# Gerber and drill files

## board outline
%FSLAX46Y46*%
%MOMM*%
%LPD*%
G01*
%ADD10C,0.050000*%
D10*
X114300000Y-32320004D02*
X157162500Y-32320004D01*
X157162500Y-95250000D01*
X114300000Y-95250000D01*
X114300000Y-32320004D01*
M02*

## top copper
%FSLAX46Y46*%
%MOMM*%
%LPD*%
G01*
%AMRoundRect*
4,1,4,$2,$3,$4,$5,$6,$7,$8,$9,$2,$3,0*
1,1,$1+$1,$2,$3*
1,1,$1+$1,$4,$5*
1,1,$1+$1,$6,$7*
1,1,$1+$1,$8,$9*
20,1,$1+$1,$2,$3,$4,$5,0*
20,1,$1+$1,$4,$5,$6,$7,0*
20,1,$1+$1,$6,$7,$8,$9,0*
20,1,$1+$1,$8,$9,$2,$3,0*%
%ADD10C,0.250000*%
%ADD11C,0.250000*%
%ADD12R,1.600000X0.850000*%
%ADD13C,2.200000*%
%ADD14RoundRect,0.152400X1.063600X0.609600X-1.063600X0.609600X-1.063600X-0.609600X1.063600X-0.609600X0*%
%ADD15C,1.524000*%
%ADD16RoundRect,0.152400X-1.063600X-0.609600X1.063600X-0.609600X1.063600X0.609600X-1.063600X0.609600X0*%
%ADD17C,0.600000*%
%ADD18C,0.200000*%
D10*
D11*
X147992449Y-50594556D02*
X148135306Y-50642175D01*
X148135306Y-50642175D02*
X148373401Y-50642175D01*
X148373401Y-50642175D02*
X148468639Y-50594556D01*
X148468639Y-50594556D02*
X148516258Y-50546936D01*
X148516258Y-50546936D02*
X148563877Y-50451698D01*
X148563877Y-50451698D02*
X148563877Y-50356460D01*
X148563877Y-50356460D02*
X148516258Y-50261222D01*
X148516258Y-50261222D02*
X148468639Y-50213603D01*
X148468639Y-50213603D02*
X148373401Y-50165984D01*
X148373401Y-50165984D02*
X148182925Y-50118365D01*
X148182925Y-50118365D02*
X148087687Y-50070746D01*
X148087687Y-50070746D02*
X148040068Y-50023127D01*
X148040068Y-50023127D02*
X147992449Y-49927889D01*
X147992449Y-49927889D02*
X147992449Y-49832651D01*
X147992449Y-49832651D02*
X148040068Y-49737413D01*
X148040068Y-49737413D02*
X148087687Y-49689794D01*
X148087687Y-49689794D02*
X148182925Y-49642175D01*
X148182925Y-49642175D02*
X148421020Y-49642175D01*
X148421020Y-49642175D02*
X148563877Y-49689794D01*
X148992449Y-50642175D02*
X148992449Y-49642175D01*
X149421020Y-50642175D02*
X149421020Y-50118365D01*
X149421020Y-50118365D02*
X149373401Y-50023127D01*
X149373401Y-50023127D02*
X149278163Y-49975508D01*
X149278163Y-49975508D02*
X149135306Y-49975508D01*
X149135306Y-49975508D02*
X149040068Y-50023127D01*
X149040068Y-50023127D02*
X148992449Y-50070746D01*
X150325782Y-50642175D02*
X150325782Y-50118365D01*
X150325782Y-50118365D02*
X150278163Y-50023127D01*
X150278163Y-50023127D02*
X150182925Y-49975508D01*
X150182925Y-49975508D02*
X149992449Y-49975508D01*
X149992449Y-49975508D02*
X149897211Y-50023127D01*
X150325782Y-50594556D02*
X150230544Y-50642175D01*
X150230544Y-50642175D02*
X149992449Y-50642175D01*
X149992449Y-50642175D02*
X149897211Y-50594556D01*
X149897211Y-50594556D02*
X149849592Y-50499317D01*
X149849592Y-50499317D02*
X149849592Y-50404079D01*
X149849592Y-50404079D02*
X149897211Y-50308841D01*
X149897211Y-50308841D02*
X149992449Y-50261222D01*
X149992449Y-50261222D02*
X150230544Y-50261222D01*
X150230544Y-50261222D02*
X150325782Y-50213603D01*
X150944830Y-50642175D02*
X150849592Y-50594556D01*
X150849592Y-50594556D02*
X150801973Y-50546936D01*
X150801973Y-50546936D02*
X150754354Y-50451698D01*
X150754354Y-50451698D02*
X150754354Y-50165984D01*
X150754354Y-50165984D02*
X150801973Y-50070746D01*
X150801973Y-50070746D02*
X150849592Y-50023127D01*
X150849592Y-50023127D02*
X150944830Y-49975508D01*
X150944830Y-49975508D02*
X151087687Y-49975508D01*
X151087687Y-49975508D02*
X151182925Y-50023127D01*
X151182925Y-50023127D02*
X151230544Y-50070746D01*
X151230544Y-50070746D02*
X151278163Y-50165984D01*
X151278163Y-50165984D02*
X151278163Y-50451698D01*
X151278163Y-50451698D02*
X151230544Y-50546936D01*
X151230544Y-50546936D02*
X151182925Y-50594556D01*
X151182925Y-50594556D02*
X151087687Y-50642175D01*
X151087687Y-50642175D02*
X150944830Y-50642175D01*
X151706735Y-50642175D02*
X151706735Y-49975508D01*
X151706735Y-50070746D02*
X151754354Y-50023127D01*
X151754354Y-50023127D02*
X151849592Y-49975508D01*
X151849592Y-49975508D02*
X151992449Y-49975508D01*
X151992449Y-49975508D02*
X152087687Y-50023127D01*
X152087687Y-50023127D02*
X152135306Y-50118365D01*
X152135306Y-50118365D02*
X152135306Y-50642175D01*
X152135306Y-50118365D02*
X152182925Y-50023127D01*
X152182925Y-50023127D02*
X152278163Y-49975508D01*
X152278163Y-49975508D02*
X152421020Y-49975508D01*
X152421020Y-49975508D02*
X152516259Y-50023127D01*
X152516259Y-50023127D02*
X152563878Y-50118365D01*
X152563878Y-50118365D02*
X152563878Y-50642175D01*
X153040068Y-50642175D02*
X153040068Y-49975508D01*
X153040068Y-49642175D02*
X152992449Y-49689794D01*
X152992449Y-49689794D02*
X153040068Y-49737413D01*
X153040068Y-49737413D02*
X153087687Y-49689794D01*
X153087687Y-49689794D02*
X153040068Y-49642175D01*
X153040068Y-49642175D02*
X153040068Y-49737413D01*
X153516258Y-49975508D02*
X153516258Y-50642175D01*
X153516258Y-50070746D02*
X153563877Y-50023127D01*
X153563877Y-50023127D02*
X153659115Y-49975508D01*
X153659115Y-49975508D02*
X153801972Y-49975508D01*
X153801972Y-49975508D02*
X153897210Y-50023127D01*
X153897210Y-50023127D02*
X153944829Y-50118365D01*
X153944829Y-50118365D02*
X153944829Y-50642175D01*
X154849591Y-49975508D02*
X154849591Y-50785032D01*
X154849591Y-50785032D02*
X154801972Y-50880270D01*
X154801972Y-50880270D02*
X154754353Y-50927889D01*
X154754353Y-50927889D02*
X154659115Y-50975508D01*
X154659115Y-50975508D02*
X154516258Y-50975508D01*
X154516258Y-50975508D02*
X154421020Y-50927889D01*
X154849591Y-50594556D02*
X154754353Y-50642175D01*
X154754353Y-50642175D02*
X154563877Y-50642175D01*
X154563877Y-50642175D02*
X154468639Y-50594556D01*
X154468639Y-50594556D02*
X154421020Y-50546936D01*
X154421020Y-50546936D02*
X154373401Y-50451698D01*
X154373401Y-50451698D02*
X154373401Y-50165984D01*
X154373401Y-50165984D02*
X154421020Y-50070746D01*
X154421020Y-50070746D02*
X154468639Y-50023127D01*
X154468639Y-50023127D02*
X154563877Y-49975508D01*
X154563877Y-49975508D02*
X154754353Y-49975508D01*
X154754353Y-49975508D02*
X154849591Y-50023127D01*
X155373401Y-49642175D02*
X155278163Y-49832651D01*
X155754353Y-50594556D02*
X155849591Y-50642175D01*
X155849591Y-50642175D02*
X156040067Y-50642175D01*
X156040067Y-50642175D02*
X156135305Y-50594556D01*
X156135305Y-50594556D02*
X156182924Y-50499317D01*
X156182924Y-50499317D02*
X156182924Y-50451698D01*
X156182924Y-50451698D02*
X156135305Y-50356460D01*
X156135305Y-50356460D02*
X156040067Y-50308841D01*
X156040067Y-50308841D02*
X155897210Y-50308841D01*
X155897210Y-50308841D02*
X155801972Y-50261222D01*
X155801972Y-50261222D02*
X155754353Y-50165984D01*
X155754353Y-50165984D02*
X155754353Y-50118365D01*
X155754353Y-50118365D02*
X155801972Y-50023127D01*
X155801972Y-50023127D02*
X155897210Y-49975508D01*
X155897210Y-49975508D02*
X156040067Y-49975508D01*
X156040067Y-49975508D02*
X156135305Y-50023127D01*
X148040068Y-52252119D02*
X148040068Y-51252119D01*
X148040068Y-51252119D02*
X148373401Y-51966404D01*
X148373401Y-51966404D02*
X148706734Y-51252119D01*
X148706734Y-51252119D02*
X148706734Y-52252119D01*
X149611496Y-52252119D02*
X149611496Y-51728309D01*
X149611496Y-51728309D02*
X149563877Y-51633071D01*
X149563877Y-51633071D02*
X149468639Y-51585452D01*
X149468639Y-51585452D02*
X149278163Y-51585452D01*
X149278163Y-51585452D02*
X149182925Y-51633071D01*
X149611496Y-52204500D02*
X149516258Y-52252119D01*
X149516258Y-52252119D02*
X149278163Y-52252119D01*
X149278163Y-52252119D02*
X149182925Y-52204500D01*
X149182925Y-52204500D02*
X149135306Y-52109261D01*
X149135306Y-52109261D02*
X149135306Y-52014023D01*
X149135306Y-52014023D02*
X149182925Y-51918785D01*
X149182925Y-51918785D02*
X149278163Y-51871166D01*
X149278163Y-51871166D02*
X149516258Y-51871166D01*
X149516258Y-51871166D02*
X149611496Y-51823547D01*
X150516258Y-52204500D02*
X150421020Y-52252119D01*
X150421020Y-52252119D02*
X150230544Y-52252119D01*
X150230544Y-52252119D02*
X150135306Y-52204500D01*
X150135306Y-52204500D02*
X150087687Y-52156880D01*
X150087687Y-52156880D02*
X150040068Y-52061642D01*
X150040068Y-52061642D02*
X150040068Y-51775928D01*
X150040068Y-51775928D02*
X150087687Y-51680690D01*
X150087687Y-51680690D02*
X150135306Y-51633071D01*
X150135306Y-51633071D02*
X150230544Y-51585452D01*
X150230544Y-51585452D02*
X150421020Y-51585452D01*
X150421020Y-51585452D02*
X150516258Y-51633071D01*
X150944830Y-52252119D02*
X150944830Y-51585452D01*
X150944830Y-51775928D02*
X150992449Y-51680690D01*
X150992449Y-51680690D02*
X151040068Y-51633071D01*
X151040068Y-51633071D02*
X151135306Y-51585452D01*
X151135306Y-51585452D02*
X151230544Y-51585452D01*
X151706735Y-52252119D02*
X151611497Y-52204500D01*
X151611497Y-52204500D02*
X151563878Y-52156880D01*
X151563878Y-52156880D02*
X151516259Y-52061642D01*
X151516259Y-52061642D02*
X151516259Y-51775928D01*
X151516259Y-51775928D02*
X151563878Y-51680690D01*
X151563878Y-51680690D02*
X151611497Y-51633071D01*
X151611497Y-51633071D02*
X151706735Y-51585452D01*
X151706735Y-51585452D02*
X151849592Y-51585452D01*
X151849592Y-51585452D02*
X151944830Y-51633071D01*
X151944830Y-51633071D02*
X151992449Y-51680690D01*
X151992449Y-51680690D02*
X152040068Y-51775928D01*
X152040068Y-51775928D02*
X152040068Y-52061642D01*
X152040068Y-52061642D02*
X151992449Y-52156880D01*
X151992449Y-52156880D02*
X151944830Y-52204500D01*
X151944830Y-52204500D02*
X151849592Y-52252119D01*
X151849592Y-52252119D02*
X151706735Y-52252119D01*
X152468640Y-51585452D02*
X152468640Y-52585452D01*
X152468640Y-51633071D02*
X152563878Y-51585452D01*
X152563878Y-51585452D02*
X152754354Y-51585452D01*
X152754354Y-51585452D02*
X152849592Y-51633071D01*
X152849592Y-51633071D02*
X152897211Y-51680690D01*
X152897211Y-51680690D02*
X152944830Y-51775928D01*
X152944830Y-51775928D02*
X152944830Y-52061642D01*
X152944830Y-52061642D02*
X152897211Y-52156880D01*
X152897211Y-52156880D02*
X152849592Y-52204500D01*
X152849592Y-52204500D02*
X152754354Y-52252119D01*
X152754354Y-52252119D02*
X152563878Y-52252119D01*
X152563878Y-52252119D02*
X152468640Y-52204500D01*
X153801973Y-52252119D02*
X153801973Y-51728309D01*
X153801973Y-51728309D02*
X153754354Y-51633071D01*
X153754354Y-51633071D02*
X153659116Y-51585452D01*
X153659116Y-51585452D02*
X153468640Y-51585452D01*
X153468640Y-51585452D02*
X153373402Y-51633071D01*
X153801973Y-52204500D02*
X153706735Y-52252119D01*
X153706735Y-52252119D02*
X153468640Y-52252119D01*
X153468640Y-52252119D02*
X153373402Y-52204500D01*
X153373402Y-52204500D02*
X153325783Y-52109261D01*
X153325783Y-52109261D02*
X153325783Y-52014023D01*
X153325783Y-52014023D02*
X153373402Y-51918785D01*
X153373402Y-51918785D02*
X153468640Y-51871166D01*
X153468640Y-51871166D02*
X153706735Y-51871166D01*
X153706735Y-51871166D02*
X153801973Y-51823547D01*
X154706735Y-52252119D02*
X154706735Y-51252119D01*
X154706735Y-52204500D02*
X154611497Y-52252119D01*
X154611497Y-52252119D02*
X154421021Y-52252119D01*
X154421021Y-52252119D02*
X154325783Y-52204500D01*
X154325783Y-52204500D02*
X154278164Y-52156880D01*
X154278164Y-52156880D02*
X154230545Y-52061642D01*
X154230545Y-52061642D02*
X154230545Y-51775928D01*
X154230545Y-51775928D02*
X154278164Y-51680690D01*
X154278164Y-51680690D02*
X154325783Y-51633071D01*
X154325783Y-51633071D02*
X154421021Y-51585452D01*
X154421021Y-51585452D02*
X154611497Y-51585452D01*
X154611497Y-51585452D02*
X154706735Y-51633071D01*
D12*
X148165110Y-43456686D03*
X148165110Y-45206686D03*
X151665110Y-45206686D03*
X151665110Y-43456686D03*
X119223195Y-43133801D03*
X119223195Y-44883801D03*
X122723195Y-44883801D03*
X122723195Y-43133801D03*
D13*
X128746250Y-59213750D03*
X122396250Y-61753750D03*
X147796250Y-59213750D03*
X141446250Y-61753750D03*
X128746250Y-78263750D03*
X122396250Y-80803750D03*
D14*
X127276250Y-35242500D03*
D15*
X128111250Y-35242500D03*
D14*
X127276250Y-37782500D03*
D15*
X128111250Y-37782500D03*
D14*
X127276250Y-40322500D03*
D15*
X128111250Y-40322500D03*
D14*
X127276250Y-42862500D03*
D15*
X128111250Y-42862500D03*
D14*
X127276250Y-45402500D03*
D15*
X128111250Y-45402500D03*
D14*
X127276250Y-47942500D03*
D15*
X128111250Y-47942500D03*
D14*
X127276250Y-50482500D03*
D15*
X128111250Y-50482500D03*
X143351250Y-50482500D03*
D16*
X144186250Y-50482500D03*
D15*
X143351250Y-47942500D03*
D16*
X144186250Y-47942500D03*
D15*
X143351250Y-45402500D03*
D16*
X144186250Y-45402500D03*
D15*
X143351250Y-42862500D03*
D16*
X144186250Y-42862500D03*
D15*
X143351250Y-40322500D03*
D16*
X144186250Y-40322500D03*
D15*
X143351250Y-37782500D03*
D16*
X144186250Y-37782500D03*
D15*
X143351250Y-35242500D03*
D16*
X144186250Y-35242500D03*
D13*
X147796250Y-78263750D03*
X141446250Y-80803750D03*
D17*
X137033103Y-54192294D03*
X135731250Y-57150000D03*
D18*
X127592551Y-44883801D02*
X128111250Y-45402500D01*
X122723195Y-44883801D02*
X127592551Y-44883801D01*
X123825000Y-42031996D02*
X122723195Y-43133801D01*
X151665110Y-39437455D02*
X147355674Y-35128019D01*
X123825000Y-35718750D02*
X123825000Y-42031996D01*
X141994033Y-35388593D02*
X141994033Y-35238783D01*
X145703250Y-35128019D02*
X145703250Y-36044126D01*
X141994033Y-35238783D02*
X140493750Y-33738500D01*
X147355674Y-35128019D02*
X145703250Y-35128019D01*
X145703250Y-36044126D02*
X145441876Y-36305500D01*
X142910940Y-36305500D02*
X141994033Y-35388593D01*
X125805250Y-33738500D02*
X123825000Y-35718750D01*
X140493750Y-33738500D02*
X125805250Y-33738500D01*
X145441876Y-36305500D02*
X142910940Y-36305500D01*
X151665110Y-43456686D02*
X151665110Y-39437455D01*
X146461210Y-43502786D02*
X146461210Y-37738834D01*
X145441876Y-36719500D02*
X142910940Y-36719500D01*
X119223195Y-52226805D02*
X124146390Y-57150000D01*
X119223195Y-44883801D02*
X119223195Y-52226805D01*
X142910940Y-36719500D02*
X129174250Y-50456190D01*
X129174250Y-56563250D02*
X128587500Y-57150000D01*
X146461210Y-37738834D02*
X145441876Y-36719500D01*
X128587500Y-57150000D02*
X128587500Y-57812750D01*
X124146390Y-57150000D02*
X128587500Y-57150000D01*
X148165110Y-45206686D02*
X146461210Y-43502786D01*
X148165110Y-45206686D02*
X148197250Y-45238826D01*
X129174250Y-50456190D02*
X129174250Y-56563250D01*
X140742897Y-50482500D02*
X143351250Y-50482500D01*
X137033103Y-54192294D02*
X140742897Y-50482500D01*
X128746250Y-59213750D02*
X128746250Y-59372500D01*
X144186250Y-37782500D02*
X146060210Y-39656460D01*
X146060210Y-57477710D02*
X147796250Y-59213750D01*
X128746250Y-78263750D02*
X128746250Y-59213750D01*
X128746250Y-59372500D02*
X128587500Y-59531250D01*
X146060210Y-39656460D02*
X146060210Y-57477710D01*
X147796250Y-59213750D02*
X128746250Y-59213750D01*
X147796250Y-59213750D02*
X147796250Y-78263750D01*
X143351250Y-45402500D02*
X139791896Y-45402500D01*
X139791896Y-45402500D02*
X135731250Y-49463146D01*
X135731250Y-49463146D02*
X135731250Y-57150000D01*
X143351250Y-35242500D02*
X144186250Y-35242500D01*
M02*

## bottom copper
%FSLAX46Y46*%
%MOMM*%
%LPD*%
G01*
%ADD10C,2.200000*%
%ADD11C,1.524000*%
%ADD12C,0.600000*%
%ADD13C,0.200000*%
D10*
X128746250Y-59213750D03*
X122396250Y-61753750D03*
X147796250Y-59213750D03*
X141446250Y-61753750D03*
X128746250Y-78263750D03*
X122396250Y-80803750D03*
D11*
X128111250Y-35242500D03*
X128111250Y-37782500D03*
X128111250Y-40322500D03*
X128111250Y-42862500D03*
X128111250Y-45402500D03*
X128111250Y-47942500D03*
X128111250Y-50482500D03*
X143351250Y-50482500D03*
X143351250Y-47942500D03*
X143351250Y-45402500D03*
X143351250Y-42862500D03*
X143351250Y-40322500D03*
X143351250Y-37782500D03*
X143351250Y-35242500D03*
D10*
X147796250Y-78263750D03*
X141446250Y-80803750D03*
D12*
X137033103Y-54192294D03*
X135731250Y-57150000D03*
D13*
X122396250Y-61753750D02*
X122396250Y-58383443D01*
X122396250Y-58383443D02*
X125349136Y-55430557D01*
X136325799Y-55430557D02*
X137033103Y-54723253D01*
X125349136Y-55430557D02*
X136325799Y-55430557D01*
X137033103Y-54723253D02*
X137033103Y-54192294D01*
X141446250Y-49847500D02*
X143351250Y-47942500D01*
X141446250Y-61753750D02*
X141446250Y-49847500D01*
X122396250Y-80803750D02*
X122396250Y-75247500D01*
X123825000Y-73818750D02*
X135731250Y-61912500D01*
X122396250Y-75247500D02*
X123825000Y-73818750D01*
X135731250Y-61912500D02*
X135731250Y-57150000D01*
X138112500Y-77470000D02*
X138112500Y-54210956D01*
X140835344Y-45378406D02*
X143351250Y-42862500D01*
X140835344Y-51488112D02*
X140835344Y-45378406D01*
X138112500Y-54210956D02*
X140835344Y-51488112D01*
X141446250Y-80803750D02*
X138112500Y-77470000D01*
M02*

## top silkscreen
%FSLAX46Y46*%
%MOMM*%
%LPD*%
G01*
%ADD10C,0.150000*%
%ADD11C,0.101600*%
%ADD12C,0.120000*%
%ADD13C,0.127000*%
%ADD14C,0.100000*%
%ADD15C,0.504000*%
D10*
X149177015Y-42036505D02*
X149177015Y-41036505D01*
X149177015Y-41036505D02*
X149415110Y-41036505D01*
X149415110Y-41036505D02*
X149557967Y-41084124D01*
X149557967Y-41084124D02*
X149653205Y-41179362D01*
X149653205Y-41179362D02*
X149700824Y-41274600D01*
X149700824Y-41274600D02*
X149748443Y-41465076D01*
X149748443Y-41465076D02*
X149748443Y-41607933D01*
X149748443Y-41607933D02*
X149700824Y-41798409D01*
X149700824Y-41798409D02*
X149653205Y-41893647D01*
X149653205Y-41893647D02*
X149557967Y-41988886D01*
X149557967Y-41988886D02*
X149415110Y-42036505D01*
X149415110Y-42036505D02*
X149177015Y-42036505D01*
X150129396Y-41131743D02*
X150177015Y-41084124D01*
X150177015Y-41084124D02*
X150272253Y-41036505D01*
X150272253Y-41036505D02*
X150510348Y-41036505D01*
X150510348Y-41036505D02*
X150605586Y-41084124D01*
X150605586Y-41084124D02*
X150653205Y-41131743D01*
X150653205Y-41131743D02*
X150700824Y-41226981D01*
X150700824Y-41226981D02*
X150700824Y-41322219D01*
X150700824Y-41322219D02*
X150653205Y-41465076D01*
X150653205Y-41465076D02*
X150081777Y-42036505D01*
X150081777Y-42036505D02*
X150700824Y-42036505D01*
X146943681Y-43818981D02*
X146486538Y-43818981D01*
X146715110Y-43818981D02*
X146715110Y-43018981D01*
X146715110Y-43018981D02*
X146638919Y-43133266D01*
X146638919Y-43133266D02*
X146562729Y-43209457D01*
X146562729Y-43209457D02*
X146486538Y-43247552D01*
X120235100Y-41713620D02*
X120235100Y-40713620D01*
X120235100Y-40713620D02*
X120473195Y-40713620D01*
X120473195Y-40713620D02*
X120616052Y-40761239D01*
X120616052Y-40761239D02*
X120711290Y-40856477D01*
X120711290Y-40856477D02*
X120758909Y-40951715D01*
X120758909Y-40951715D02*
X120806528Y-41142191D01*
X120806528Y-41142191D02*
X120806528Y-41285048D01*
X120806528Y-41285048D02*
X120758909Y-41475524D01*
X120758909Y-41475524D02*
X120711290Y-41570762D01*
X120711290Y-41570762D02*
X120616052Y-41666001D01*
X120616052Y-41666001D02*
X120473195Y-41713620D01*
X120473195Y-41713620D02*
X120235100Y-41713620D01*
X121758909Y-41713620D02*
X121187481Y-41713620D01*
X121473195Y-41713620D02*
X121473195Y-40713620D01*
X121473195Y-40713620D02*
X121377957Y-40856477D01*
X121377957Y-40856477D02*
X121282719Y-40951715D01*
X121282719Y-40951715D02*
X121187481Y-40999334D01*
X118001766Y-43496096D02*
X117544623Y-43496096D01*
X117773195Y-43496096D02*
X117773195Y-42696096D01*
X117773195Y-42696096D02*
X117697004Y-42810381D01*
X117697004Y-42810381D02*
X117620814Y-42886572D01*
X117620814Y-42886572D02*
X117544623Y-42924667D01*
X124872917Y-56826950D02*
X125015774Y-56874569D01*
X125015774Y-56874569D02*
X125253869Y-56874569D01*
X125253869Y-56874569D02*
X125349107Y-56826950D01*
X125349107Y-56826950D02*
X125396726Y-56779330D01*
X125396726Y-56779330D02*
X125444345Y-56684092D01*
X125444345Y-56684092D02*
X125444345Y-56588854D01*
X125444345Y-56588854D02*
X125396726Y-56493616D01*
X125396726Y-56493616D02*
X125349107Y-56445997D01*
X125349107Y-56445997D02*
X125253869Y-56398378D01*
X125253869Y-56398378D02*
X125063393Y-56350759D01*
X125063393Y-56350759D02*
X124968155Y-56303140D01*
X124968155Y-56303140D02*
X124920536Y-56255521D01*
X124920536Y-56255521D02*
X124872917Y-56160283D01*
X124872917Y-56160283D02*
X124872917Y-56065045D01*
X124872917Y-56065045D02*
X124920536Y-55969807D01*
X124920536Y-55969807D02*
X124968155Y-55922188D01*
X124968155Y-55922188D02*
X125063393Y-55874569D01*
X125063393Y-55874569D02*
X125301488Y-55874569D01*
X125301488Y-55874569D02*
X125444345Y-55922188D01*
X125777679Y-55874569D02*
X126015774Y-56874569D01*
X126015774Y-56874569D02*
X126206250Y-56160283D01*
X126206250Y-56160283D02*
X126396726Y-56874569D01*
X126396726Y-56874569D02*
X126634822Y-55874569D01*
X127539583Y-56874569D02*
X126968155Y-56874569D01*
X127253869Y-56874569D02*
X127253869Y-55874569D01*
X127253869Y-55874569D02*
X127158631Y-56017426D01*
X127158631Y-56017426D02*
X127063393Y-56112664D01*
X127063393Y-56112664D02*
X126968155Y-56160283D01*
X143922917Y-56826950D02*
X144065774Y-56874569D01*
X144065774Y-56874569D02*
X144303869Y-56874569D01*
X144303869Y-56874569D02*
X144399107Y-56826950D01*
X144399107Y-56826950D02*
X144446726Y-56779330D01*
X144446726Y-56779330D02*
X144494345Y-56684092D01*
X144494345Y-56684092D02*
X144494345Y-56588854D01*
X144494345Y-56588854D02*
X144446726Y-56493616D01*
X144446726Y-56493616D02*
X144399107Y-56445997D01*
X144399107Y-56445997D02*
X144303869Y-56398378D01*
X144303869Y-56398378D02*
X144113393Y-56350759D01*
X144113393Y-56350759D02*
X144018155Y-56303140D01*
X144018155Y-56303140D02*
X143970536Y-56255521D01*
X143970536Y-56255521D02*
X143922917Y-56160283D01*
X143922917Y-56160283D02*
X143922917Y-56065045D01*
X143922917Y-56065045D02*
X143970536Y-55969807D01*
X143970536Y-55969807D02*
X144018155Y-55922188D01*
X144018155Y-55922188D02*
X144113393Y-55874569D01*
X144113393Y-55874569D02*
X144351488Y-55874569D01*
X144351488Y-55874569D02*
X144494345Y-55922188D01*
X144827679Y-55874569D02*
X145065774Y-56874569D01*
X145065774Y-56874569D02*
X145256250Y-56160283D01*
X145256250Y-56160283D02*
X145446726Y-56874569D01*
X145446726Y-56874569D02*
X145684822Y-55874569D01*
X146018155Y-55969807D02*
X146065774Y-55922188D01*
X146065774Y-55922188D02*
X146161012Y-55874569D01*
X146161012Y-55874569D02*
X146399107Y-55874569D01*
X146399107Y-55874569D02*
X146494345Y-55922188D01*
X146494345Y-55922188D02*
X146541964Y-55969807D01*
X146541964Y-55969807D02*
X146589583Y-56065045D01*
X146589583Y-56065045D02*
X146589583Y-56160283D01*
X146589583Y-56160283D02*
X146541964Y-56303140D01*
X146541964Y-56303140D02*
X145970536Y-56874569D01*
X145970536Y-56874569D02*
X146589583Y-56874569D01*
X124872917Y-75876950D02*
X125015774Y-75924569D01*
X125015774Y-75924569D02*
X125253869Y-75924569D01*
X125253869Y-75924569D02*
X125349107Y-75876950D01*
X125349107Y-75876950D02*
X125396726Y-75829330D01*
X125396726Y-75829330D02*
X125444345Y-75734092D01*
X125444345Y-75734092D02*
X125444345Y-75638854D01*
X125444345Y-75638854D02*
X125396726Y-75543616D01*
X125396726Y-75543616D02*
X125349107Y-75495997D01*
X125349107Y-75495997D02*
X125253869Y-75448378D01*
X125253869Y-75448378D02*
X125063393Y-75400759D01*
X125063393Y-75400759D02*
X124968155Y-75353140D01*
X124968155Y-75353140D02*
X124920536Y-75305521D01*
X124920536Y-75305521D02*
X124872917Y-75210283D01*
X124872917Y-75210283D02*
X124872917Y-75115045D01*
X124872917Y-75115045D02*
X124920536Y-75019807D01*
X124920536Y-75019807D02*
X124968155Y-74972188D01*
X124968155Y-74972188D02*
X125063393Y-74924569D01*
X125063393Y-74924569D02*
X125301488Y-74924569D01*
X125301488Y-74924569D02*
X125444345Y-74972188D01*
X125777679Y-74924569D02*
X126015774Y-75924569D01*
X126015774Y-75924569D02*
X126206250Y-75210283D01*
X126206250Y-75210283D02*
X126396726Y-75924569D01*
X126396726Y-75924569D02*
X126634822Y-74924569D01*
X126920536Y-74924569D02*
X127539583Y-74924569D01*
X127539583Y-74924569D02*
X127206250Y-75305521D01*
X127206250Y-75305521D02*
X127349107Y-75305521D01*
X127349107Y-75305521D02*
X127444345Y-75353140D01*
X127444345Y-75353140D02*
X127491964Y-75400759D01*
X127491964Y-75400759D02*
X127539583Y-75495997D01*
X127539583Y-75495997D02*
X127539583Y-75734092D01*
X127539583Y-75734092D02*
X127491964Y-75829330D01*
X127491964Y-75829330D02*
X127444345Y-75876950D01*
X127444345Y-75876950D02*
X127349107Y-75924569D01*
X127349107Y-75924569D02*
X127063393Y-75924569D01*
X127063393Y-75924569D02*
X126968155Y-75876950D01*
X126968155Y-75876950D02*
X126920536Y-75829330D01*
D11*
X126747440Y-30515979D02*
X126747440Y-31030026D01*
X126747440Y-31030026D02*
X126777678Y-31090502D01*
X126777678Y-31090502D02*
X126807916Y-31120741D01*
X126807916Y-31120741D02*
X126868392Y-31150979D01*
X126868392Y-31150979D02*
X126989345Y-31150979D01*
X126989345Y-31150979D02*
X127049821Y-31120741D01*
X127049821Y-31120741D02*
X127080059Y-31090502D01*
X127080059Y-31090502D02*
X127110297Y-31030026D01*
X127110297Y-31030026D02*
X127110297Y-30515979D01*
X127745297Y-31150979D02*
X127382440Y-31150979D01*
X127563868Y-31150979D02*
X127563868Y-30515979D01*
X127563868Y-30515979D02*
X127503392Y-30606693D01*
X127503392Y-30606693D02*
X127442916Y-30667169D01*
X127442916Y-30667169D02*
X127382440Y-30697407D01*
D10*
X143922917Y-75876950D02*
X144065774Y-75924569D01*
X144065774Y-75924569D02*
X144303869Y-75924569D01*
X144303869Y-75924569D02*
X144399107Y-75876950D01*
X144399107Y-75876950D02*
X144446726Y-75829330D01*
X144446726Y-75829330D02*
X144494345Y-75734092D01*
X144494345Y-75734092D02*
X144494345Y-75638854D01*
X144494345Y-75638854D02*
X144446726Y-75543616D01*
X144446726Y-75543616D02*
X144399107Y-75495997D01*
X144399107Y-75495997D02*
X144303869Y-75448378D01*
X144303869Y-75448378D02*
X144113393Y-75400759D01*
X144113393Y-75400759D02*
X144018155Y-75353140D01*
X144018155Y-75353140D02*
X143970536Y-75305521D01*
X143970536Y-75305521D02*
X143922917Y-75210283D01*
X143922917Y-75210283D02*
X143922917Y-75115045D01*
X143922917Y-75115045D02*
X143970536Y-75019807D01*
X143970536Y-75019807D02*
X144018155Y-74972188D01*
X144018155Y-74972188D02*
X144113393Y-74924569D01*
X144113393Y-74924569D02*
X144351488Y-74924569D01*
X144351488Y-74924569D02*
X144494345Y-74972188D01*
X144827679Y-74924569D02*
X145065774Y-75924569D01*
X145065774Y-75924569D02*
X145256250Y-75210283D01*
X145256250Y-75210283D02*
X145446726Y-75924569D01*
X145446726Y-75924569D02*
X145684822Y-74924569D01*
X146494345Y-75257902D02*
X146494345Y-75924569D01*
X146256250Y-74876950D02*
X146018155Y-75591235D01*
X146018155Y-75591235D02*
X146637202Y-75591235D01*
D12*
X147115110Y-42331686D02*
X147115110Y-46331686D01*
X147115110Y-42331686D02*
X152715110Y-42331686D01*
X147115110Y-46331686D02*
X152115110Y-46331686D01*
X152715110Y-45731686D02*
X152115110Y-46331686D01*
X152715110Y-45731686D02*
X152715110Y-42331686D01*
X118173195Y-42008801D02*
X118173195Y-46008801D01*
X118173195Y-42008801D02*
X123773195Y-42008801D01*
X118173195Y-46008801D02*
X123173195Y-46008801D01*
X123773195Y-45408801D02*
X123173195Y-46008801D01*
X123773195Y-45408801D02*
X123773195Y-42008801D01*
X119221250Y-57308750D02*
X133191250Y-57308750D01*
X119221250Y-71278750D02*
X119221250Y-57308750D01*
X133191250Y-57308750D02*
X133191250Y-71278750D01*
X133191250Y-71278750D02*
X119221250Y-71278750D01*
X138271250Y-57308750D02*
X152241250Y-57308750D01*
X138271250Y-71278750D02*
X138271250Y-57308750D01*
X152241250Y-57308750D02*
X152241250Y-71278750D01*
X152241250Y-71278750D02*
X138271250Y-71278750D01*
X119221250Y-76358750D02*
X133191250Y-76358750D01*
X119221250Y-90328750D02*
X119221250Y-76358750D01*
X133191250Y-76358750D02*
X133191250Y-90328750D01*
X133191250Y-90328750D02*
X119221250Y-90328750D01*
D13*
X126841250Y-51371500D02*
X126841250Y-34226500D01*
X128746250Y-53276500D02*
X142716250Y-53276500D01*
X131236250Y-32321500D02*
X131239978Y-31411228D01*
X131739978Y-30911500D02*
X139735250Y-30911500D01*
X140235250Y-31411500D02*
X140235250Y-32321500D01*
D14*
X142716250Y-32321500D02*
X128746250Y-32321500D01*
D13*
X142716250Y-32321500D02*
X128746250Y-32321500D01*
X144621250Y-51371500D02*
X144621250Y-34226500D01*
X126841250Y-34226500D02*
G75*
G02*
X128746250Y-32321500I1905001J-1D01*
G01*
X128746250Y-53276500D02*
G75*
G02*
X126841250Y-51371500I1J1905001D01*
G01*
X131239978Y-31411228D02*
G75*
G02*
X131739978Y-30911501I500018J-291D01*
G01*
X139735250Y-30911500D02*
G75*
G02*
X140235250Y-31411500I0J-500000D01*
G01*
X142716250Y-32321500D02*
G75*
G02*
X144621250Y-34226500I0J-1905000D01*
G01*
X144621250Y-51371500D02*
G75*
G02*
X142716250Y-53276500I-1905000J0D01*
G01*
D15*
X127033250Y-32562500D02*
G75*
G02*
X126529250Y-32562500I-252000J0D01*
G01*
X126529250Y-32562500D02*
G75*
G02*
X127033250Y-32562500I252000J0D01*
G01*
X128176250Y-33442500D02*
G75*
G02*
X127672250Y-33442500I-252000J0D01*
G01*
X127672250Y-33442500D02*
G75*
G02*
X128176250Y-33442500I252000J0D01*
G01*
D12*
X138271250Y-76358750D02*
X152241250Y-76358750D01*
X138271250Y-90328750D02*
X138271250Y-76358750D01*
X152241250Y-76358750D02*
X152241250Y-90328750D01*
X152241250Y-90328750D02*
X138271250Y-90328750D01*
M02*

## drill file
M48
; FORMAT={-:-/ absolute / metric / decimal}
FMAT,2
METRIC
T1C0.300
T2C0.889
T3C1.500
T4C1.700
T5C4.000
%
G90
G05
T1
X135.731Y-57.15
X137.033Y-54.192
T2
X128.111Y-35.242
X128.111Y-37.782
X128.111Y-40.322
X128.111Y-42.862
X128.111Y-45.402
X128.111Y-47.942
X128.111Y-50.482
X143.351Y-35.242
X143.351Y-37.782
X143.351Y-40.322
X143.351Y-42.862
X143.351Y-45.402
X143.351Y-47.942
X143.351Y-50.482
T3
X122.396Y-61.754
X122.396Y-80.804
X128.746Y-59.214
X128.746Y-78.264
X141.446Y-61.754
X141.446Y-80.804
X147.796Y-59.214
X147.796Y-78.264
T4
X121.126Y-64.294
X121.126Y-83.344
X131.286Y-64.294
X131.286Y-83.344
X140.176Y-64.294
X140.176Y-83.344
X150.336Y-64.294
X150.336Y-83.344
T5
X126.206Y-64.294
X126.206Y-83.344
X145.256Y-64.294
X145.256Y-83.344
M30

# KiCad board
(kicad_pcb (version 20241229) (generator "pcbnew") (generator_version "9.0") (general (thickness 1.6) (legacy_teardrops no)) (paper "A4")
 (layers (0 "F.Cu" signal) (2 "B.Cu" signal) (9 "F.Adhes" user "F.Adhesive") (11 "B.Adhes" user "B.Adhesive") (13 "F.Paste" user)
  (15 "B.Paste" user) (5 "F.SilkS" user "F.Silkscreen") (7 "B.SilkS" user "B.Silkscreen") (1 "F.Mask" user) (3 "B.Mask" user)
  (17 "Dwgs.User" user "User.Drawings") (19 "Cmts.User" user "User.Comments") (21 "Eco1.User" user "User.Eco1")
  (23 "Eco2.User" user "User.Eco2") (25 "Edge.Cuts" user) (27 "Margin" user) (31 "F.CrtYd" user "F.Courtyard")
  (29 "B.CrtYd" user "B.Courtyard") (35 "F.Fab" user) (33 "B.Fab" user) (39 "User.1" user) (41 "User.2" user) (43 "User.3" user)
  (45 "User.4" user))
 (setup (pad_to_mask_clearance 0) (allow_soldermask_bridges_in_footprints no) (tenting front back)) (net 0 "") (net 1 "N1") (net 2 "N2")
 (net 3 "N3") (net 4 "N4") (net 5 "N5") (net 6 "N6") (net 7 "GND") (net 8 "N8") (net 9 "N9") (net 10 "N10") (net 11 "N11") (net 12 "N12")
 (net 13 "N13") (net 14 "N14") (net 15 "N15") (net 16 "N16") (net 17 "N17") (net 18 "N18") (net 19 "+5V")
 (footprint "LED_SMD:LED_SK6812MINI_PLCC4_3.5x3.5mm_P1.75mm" (layer "F.Cu") (at 149.91511 44.331686)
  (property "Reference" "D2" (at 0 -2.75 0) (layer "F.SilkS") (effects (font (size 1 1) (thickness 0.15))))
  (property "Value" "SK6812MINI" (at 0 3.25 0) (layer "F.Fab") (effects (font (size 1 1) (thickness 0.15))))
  (fp_line (start -2.8 -2) (end -2.8 2) (stroke (width 0.12) (type default)) (layer "F.SilkS"))
  (fp_line (start -2.8 -2) (end 2.8 -2) (stroke (width 0.12) (type solid)) (layer "F.SilkS"))
  (fp_line (start -2.8 2) (end 2.2 2) (stroke (width 0.12) (type solid)) (layer "F.SilkS"))
  (fp_line (start 2.8 1.4) (end 2.2 2) (stroke (width 0.12) (type default)) (layer "F.SilkS"))
  (fp_line (start 2.8 1.4) (end 2.8 -2) (stroke (width 0.12) (type solid)) (layer "F.SilkS"))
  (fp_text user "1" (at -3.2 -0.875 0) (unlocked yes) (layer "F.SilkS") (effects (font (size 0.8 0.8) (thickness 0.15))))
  (pad "1" smd rect (at -1.75 -0.875) (size 1.6 0.85) (layers "F.Cu" "F.Mask" "F.Paste") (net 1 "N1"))
  (pad "2" smd rect (at -1.75 0.875) (size 1.6 0.85) (layers "F.Cu" "F.Mask" "F.Paste") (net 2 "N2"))
  (pad "3" smd rect (at 1.75 0.875) (size 1.6 0.85) (layers "F.Cu" "F.Mask" "F.Paste") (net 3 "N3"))
  (pad "4" smd rect (at 1.75 -0.875) (size 1.6 0.85) (layers "F.Cu" "F.Mask" "F.Paste") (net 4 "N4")))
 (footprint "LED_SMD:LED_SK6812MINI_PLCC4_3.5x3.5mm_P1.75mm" (layer "F.Cu") (at 120.973195 44.008801)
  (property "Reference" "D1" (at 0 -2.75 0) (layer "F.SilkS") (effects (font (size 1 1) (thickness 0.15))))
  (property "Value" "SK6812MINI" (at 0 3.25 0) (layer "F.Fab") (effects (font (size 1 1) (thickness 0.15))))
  (fp_line (start -2.8 -2) (end -2.8 2) (stroke (width 0.12) (type default)) (layer "F.SilkS"))
  (fp_line (start -2.8 -2) (end 2.8 -2) (stroke (width 0.12) (type solid)) (layer "F.SilkS"))
  (fp_line (start -2.8 2) (end 2.2 2) (stroke (width 0.12) (type solid)) (layer "F.SilkS"))
  (fp_line (start 2.8 1.4) (end 2.2 2) (stroke (width 0.12) (type default)) (layer "F.SilkS"))
  (fp_line (start 2.8 1.4) (end 2.8 -2) (stroke (width 0.12) (type solid)) (layer "F.SilkS"))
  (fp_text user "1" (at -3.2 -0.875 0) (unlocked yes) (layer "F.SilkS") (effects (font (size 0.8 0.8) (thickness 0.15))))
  (pad "1" smd rect (at -1.75 -0.875) (size 1.6 0.85) (layers "F.Cu" "F.Mask" "F.Paste") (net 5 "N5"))
  (pad "2" smd rect (at -1.75 0.875) (size 1.6 0.85) (layers "F.Cu" "F.Mask" "F.Paste") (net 2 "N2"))
  (pad "3" smd rect (at 1.75 0.875) (size 1.6 0.85) (layers "F.Cu" "F.Mask" "F.Paste") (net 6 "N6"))
  (pad "4" smd rect (at 1.75 -0.875) (size 1.6 0.85) (layers "F.Cu" "F.Mask" "F.Paste") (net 4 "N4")))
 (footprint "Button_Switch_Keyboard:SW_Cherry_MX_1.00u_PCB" (layer "F.Cu") (at 128.74625 59.21375)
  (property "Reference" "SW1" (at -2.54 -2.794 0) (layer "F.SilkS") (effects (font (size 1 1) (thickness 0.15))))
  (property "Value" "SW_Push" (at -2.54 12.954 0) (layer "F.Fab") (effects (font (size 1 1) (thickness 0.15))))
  (fp_line (start -9.525 -1.905) (end 4.445 -1.905) (stroke (width 0.12) (type solid)) (layer "F.SilkS"))
  (fp_line (start -9.525 12.065) (end -9.525 -1.905) (stroke (width 0.12) (type solid)) (layer "F.SilkS"))
  (fp_line (start 4.445 -1.905) (end 4.445 12.065) (stroke (width 0.12) (type solid)) (layer "F.SilkS"))
  (fp_line (start 4.445 12.065) (end -9.525 12.065) (stroke (width 0.12) (type solid)) (layer "F.SilkS"))
  (pad "" np_thru_hole circle (at -7.62 5.08) (size 1.7 1.7) (drill 1.7) (layers "*.Cu" "*.Mask"))
  (pad "" np_thru_hole circle (at -2.54 5.08) (size 4 4) (drill 4) (layers "*.Cu" "*.Mask"))
  (pad "" np_thru_hole circle (at 2.54 5.08) (size 1.7 1.7) (drill 1.7) (layers "*.Cu" "*.Mask"))
  (pad "1" thru_hole circle (at 0 0) (size 2.2 2.2) (drill 1.5) (layers "*.Cu" "*.Mask") (remove_unused_layers no) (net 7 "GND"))
  (pad "2" thru_hole circle (at -6.35 2.54) (size 2.2 2.2) (drill 1.5) (layers "*.Cu" "*.Mask") (remove_unused_layers no) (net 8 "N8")))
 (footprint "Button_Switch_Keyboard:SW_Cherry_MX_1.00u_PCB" (layer "F.Cu") (at 147.79625 59.21375)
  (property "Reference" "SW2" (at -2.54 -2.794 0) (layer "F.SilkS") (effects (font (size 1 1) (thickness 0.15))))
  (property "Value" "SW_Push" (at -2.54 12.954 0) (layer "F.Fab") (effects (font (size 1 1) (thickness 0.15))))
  (fp_line (start -9.525 -1.905) (end 4.445 -1.905) (stroke (width 0.12) (type solid)) (layer "F.SilkS"))
  (fp_line (start -9.525 12.065) (end -9.525 -1.905) (stroke (width 0.12) (type solid)) (layer "F.SilkS"))
  (fp_line (start 4.445 -1.905) (end 4.445 12.065) (stroke (width 0.12) (type solid)) (layer "F.SilkS"))
  (fp_line (start 4.445 12.065) (end -9.525 12.065) (stroke (width 0.12) (type solid)) (layer "F.SilkS"))
  (pad "" np_thru_hole circle (at -7.62 5.08) (size 1.7 1.7) (drill 1.7) (layers "*.Cu" "*.Mask"))
  (pad "" np_thru_hole circle (at -2.54 5.08) (size 4 4) (drill 4) (layers "*.Cu" "*.Mask"))
  (pad "" np_thru_hole circle (at 2.54 5.08) (size 1.7 1.7) (drill 1.7) (layers "*.Cu" "*.Mask"))
  (pad "1" thru_hole circle (at 0 0) (size 2.2 2.2) (drill 1.5) (layers "*.Cu" "*.Mask") (remove_unused_layers no) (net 7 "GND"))
  (pad "2" thru_hole circle (at -6.35 2.54) (size 2.2 2.2) (drill 1.5) (layers "*.Cu" "*.Mask") (remove_unused_layers no) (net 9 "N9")))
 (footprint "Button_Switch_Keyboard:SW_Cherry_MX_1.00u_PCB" (layer "F.Cu") (at 128.74625 78.26375)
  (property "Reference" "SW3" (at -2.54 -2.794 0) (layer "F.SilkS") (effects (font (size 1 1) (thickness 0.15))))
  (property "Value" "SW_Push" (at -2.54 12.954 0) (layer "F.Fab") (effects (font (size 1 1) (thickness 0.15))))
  (fp_line (start -9.525 -1.905) (end 4.445 -1.905) (stroke (width 0.12) (type solid)) (layer "F.SilkS"))
  (fp_line (start -9.525 12.065) (end -9.525 -1.905) (stroke (width 0.12) (type solid)) (layer "F.SilkS"))
  (fp_line (start 4.445 -1.905) (end 4.445 12.065) (stroke (width 0.12) (type solid)) (layer "F.SilkS"))
  (fp_line (start 4.445 12.065) (end -9.525 12.065) (stroke (width 0.12) (type solid)) (layer "F.SilkS"))
  (pad "" np_thru_hole circle (at -7.62 5.08) (size 1.7 1.7) (drill 1.7) (layers "*.Cu" "*.Mask"))
  (pad "" np_thru_hole circle (at -2.54 5.08) (size 4 4) (drill 4) (layers "*.Cu" "*.Mask"))
  (pad "" np_thru_hole circle (at 2.54 5.08) (size 1.7 1.7) (drill 1.7) (layers "*.Cu" "*.Mask"))
  (pad "1" thru_hole circle (at 0 0) (size 2.2 2.2) (drill 1.5) (layers "*.Cu" "*.Mask") (remove_unused_layers no) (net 7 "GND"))
  (pad "2" thru_hole circle (at -6.35 2.54) (size 2.2 2.2) (drill 1.5) (layers "*.Cu" "*.Mask") (remove_unused_layers no) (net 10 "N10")))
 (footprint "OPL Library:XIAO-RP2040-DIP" (layer "F.Cu") (at 135.73125 42.8625)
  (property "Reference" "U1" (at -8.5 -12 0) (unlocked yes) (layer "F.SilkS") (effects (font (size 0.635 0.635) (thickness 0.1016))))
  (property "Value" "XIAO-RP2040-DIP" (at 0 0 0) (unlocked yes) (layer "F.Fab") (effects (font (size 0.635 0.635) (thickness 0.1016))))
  (fp_line (start -8.89 8.509) (end -8.89 -8.636) (stroke (width 0.127) (type solid)) (layer "F.SilkS"))
  (fp_line (start -6.985 10.414) (end 6.985 10.414) (stroke (width 0.127) (type solid)) (layer "F.SilkS"))
  (fp_line (start -4.495 -10.541) (end -4.491272 -11.451272) (stroke (width 0.127) (type solid)) (layer "F.SilkS"))
  (fp_line (start -3.991272 -11.951) (end 4.004 -11.951) (stroke (width 0.127) (type solid)) (layer "F.SilkS"))
  (fp_line (start 4.504 -11.451) (end 4.504 -10.541) (stroke (width 0.127) (type solid)) (layer "F.SilkS"))
  (fp_line (start 6.985 -10.541) (end -6.985 -10.541) (stroke (width 0.1) (type solid)) (layer "F.SilkS"))
  (fp_line (start 6.985 -10.541) (end -6.985 -10.541) (stroke (width 0.127) (type solid)) (layer "F.SilkS"))
  (fp_line (start 8.89 8.509) (end 8.89 -8.636) (stroke (width 0.127) (type solid)) (layer "F.SilkS"))
  (fp_arc (start -8.89 -8.636) (mid -8.332038 -9.983038) (end -6.985 -10.541) (stroke (width 0.127) (type solid)) (layer "F.SilkS"))
  (fp_arc (start -6.985 10.414) (mid -8.332038 9.856038) (end -8.89 8.509) (stroke (width 0.127) (type solid)) (layer "F.SilkS"))
  (fp_arc (start -4.491272 -11.451272) (mid -4.344728 -11.80464) (end -3.991272 -11.951) (stroke (width 0.127) (type default))
   (layer "F.SilkS"))
  (fp_arc (start 4.004 -11.951) (mid 4.357553 -11.804553) (end 4.504 -11.451) (stroke (width 0.127) (type default)) (layer "F.SilkS"))
  (fp_arc (start 6.985 -10.541) (mid 8.332038 -9.983038) (end 8.89 -8.636) (stroke (width 0.127) (type solid)) (layer "F.SilkS"))
  (fp_arc (start 8.89 8.509) (mid 8.332038 9.856038) (end 6.985 10.414) (stroke (width 0.127) (type solid)) (layer "F.SilkS"))
  (fp_circle (center -8.95 -10.3) (end -8.95 -10.554) (stroke (width 0.5) (type solid)) (fill yes) (layer "F.SilkS"))
  (fp_circle (center -7.807 -9.42) (end -7.807 -9.674) (stroke (width 0.5) (type solid)) (fill yes) (layer "F.SilkS"))
  (pad "1" smd roundrect (at -8.455 -7.62 180) (size 2.432 1.524) (layers "F.Cu" "F.Mask") (roundrect_rratio 0.1) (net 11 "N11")
   (thermal_bridge_angle 45))
  (pad "1" thru_hole circle (at -7.62 -7.62 180) (size 1.524 1.524) (drill 0.889) (layers "*.Cu" "*.Mask") (remove_unused_layers no)
   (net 11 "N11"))
  (pad "2" smd roundrect (at -8.455 -5.08 180) (size 2.432 1.524) (layers "F.Cu" "F.Mask") (roundrect_rratio 0.1) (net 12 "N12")
   (thermal_bridge_angle 45))
  (pad "2" thru_hole circle (at -7.62 -5.08 180) (size 1.524 1.524) (drill 0.889) (layers "*.Cu" "*.Mask") (remove_unused_layers no)
   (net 12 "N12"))
  (pad "3" smd roundrect (at -8.455 -2.54 180) (size 2.432 1.524) (layers "F.Cu" "F.Mask") (roundrect_rratio 0.1) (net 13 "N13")
   (thermal_bridge_angle 45))
  (pad "3" thru_hole circle (at -7.62 -2.54 180) (size 1.524 1.524) (drill 0.889) (layers "*.Cu" "*.Mask") (remove_unused_layers no)
   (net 13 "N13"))
  (pad "4" smd roundrect (at -8.455 0 180) (size 2.432 1.524) (layers "F.Cu" "F.Mask") (roundrect_rratio 0.1) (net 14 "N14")
   (thermal_bridge_angle 45))
  (pad "4" thru_hole circle (at -7.62 0 180) (size 1.524 1.524) (drill 0.889) (layers "*.Cu" "*.Mask") (remove_unused_layers no)
   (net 14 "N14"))
  (pad "5" smd roundrect (at -8.455 2.54 180) (size 2.432 1.524) (layers "F.Cu" "F.Mask") (roundrect_rratio 0.1) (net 6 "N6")
   (thermal_bridge_angle 45))
  (pad "5" thru_hole circle (at -7.62 2.54 180) (size 1.524 1.524) (drill 0.889) (layers "*.Cu" "*.Mask") (remove_unused_layers no)
   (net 6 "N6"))
  (pad "6" smd roundrect (at -8.455 5.08 180) (size 2.432 1.524) (layers "F.Cu" "F.Mask") (roundrect_rratio 0.1) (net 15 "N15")
   (thermal_bridge_angle 45))
  (pad "6" thru_hole circle (at -7.62 5.08 180) (size 1.524 1.524) (drill 0.889) (layers "*.Cu" "*.Mask") (remove_unused_layers no)
   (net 15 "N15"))
  (pad "7" smd roundrect (at -8.455 7.62 180) (size 2.432 1.524) (layers "F.Cu" "F.Mask") (roundrect_rratio 0.1) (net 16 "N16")
   (thermal_bridge_angle 45))
  (pad "7" thru_hole circle (at -7.62 7.62 180) (size 1.524 1.524) (drill 0.889) (layers "*.Cu" "*.Mask") (remove_unused_layers no)
   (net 16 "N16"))
  (pad "8" thru_hole circle (at 7.62 7.62) (size 1.524 1.524) (drill 0.889) (layers "*.Cu" "*.Mask") (remove_unused_layers no) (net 8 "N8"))
  (pad "8" smd roundrect (at 8.455 7.62) (size 2.432 1.524) (layers "F.Cu" "F.Mask") (roundrect_rratio 0.1) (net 8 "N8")
   (thermal_bridge_angle 45))
  (pad "9" thru_hole circle (at 7.62 5.08) (size 1.524 1.524) (drill 0.889) (layers "*.Cu" "*.Mask") (remove_unused_layers no) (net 9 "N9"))
  (pad "9" smd roundrect (at 8.455 5.08) (size 2.432 1.524) (layers "F.Cu" "F.Mask") (roundrect_rratio 0.1) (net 9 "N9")
   (thermal_bridge_angle 45))
  (pad "10" thru_hole circle (at 7.62 2.54) (size 1.524 1.524) (drill 0.889) (layers "*.Cu" "*.Mask") (remove_unused_layers no)
   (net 10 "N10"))
  (pad "10" smd roundrect (at 8.455 2.54) (size 2.432 1.524) (layers "F.Cu" "F.Mask") (roundrect_rratio 0.1) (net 10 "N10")
   (thermal_bridge_angle 45))
  (pad "11" thru_hole circle (at 7.62 0) (size 1.524 1.524) (drill 0.889) (layers "*.Cu" "*.Mask") (remove_unused_layers no) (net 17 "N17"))
  (pad "11" smd roundrect (at 8.455 0) (size 2.432 1.524) (layers "F.Cu" "F.Mask") (roundrect_rratio 0.1) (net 17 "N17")
   (thermal_bridge_angle 45))
  (pad "12" thru_hole circle (at 7.62 -2.54) (size 1.524 1.524) (drill 0.889) (layers "*.Cu" "*.Mask") (remove_unused_layers no)
   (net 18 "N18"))
  (pad "12" smd roundrect (at 8.455 -2.54) (size 2.432 1.524) (layers "F.Cu" "F.Mask") (roundrect_rratio 0.1) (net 18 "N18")
   (thermal_bridge_angle 45))
  (pad "13" thru_hole circle (at 7.62 -5.08) (size 1.524 1.524) (drill 0.889) (layers "*.Cu" "*.Mask") (remove_unused_layers no)
   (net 7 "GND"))
  (pad "13" smd roundrect (at 8.455 -5.08) (size 2.432 1.524) (layers "F.Cu" "F.Mask") (roundrect_rratio 0.1) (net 7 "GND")
   (thermal_bridge_angle 45))
  (pad "14" thru_hole circle (at 7.62 -7.62) (size 1.524 1.524) (drill 0.889) (layers "*.Cu" "*.Mask") (remove_unused_layers no)
   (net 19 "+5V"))
  (pad "14" smd roundrect (at 8.455 -7.62) (size 2.432 1.524) (layers "F.Cu" "F.Mask") (roundrect_rratio 0.1) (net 19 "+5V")
   (thermal_bridge_angle 45)))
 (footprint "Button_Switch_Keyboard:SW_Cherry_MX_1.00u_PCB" (layer "F.Cu") (at 147.79625 78.26375)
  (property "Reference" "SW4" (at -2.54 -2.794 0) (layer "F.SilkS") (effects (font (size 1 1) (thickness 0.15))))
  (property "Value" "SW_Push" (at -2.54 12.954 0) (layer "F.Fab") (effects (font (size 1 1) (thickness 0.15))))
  (fp_line (start -9.525 -1.905) (end 4.445 -1.905) (stroke (width 0.12) (type solid)) (layer "F.SilkS"))
  (fp_line (start -9.525 12.065) (end -9.525 -1.905) (stroke (width 0.12) (type solid)) (layer "F.SilkS"))
  (fp_line (start 4.445 -1.905) (end 4.445 12.065) (stroke (width 0.12) (type solid)) (layer "F.SilkS"))
  (fp_line (start 4.445 12.065) (end -9.525 12.065) (stroke (width 0.12) (type solid)) (layer "F.SilkS"))
  (pad "" np_thru_hole circle (at -7.62 5.08) (size 1.7 1.7) (drill 1.7) (layers "*.Cu" "*.Mask"))
  (pad "" np_thru_hole circle (at -2.54 5.08) (size 4 4) (drill 4) (layers "*.Cu" "*.Mask"))
  (pad "" np_thru_hole circle (at 2.54 5.08) (size 1.7 1.7) (drill 1.7) (layers "*.Cu" "*.Mask"))
  (pad "1" thru_hole circle (at 0 0) (size 2.2 2.2) (drill 1.5) (layers "*.Cu" "*.Mask") (remove_unused_layers no) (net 7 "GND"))
  (pad "2" thru_hole circle (at -6.35 2.54) (size 2.2 2.2) (drill 1.5) (layers "*.Cu" "*.Mask") (remove_unused_layers no) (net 17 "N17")))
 (gr_rect (start 114.3 32.320004) (end 157.1625 95.25) (stroke (width 0.05) (type default)) (fill no) (layer "Edge.Cuts"))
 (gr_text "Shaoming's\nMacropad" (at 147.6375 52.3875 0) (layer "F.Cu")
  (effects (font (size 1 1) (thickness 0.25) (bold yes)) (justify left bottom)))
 (segment (start 127.592551 44.883801) (end 128.11125 45.4025) (width 0.2) (layer "F.Cu") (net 6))
 (segment (start 122.723195 44.883801) (end 127.592551 44.883801) (width 0.2) (layer "F.Cu") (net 6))
 (segment (start 123.825 42.031996) (end 122.723195 43.133801) (width 0.2) (layer "F.Cu") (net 4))
 (segment (start 151.66511 39.437455) (end 147.355674 35.128019) (width 0.2) (layer "F.Cu") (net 4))
 (segment (start 123.825 35.71875) (end 123.825 42.031996) (width 0.2) (layer "F.Cu") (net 4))
 (segment (start 141.994033 35.388593) (end 141.994033 35.238783) (width 0.2) (layer "F.Cu") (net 4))
 (segment (start 145.70325 35.128019) (end 145.70325 36.044126) (width 0.2) (layer "F.Cu") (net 4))
 (segment (start 141.994033 35.238783) (end 140.49375 33.7385) (width 0.2) (layer "F.Cu") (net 4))
 (segment (start 147.355674 35.128019) (end 145.70325 35.128019) (width 0.2) (layer "F.Cu") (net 4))
 (segment (start 145.70325 36.044126) (end 145.441876 36.3055) (width 0.2) (layer "F.Cu") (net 4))
 (segment (start 142.91094 36.3055) (end 141.994033 35.388593) (width 0.2) (layer "F.Cu") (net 4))
 (segment (start 125.80525 33.7385) (end 123.825 35.71875) (width 0.2) (layer "F.Cu") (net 4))
 (segment (start 140.49375 33.7385) (end 125.80525 33.7385) (width 0.2) (layer "F.Cu") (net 4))
 (segment (start 145.441876 36.3055) (end 142.91094 36.3055) (width 0.2) (layer "F.Cu") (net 4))
 (segment (start 151.66511 43.456686) (end 151.66511 39.437455) (width 0.2) (layer "F.Cu") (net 4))
 (segment (start 146.46121 43.502786) (end 146.46121 37.738834) (width 0.2) (layer "F.Cu") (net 2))
 (segment (start 145.441876 36.7195) (end 142.91094 36.7195) (width 0.2) (layer "F.Cu") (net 2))
 (segment (start 119.223195 52.226805) (end 124.14639 57.15) (width 0.2) (layer "F.Cu") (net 2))
 (segment (start 119.223195 44.883801) (end 119.223195 52.226805) (width 0.2) (layer "F.Cu") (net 2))
 (segment (start 142.91094 36.7195) (end 129.17425 50.45619) (width 0.2) (layer "F.Cu") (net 2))
 (segment (start 129.17425 56.56325) (end 128.5875 57.15) (width 0.2) (layer "F.Cu") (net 2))
 (segment (start 146.46121 37.738834) (end 145.441876 36.7195) (width 0.2) (layer "F.Cu") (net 2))
 (segment (start 128.5875 57.15) (end 128.5875 57.81275) (width 0.2) (layer "F.Cu") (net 2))
 (segment (start 124.14639 57.15) (end 128.5875 57.15) (width 0.2) (layer "F.Cu") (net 2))
 (segment (start 148.16511 45.206686) (end 146.46121 43.502786) (width 0.2) (layer "F.Cu") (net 2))
 (segment (start 148.16511 45.206686) (end 148.19725 45.238826) (width 0.2) (layer "F.Cu") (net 2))
 (segment (start 129.17425 50.45619) (end 129.17425 56.56325) (width 0.2) (layer "F.Cu") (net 2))
 (segment (start 140.742897 50.4825) (end 143.35125 50.4825) (width 0.2) (layer "F.Cu") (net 8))
 (segment (start 137.033103 54.192294) (end 140.742897 50.4825) (width 0.2) (layer "F.Cu") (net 8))
 (via (at 137.033103 54.192294) (size 0.6) (drill 0.3) (layers "F.Cu" "B.Cu") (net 8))
 (segment (start 122.39625 61.75375) (end 122.39625 58.383443) (width 0.2) (layer "B.Cu") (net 8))
 (segment (start 122.39625 58.383443) (end 125.349136 55.430557) (width 0.2) (layer "B.Cu") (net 8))
 (segment (start 136.325799 55.430557) (end 137.033103 54.723253) (width 0.2) (layer "B.Cu") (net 8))
 (segment (start 125.349136 55.430557) (end 136.325799 55.430557) (width 0.2) (layer "B.Cu") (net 8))
 (segment (start 137.033103 54.723253) (end 137.033103 54.192294) (width 0.2) (layer "B.Cu") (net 8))
 (segment (start 128.74625 59.21375) (end 128.74625 59.3725) (width 0.2) (layer "F.Cu") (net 7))
 (segment (start 144.18625 37.7825) (end 146.06021 39.65646) (width 0.2) (layer "F.Cu") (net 7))
 (segment (start 146.06021 57.47771) (end 147.79625 59.21375) (width 0.2) (layer "F.Cu") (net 7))
 (segment (start 128.74625 78.26375) (end 128.74625 59.21375) (width 0.2) (layer "F.Cu") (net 7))
 (segment (start 128.74625 59.3725) (end 128.5875 59.53125) (width 0.2) (layer "F.Cu") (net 7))
 (segment (start 146.06021 39.65646) (end 146.06021 57.47771) (width 0.2) (layer "F.Cu") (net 7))
 (segment (start 147.79625 59.21375) (end 128.74625 59.21375) (width 0.2) (layer "F.Cu") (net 7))
 (segment (start 147.79625 59.21375) (end 147.79625 78.26375) (width 0.2) (layer "F.Cu") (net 7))
 (segment (start 141.44625 49.8475) (end 143.35125 47.9425) (width 0.2) (layer "B.Cu") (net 9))
 (segment (start 141.44625 61.75375) (end 141.44625 49.8475) (width 0.2) (layer "B.Cu") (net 9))
 (segment (start 143.35125 45.4025) (end 139.791896 45.4025) (width 0.2) (layer "F.Cu") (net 10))
 (segment (start 139.791896 45.4025) (end 135.73125 49.463146) (width 0.2) (layer "F.Cu") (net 10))
 (segment (start 135.73125 49.463146) (end 135.73125 57.15) (width 0.2) (layer "F.Cu") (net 10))
 (via (at 135.73125 57.15) (size 0.6) (drill 0.3) (layers "F.Cu" "B.Cu") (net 10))
 (segment (start 122.39625 80.80375) (end 122.39625 75.2475) (width 0.2) (layer "B.Cu") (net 10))
 (segment (start 123.825 73.81875) (end 135.73125 61.9125) (width 0.2) (layer "B.Cu") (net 10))
 (segment (start 122.39625 75.2475) (end 123.825 73.81875) (width 0.2) (layer "B.Cu") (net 10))
 (segment (start 135.73125 61.9125) (end 135.73125 57.15) (width 0.2) (layer "B.Cu") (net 10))
 (segment (start 138.1125 77.47) (end 138.1125 54.210956) (width 0.2) (layer "B.Cu") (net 17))
 (segment (start 140.835344 45.378406) (end 143.35125 42.8625) (width 0.2) (layer "B.Cu") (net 17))
 (segment (start 140.835344 51.488112) (end 140.835344 45.378406) (width 0.2) (layer "B.Cu") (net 17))
 (segment (start 138.1125 54.210956) (end 140.835344 51.488112) (width 0.2) (layer "B.Cu") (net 17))
 (segment (start 141.44625 80.80375) (end 138.1125 77.47) (width 0.2) (layer "B.Cu") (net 17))
 (segment (start 143.35125 35.2425) (end 144.18625 35.2425) (width 0.2) (layer "F.Cu") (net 19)))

